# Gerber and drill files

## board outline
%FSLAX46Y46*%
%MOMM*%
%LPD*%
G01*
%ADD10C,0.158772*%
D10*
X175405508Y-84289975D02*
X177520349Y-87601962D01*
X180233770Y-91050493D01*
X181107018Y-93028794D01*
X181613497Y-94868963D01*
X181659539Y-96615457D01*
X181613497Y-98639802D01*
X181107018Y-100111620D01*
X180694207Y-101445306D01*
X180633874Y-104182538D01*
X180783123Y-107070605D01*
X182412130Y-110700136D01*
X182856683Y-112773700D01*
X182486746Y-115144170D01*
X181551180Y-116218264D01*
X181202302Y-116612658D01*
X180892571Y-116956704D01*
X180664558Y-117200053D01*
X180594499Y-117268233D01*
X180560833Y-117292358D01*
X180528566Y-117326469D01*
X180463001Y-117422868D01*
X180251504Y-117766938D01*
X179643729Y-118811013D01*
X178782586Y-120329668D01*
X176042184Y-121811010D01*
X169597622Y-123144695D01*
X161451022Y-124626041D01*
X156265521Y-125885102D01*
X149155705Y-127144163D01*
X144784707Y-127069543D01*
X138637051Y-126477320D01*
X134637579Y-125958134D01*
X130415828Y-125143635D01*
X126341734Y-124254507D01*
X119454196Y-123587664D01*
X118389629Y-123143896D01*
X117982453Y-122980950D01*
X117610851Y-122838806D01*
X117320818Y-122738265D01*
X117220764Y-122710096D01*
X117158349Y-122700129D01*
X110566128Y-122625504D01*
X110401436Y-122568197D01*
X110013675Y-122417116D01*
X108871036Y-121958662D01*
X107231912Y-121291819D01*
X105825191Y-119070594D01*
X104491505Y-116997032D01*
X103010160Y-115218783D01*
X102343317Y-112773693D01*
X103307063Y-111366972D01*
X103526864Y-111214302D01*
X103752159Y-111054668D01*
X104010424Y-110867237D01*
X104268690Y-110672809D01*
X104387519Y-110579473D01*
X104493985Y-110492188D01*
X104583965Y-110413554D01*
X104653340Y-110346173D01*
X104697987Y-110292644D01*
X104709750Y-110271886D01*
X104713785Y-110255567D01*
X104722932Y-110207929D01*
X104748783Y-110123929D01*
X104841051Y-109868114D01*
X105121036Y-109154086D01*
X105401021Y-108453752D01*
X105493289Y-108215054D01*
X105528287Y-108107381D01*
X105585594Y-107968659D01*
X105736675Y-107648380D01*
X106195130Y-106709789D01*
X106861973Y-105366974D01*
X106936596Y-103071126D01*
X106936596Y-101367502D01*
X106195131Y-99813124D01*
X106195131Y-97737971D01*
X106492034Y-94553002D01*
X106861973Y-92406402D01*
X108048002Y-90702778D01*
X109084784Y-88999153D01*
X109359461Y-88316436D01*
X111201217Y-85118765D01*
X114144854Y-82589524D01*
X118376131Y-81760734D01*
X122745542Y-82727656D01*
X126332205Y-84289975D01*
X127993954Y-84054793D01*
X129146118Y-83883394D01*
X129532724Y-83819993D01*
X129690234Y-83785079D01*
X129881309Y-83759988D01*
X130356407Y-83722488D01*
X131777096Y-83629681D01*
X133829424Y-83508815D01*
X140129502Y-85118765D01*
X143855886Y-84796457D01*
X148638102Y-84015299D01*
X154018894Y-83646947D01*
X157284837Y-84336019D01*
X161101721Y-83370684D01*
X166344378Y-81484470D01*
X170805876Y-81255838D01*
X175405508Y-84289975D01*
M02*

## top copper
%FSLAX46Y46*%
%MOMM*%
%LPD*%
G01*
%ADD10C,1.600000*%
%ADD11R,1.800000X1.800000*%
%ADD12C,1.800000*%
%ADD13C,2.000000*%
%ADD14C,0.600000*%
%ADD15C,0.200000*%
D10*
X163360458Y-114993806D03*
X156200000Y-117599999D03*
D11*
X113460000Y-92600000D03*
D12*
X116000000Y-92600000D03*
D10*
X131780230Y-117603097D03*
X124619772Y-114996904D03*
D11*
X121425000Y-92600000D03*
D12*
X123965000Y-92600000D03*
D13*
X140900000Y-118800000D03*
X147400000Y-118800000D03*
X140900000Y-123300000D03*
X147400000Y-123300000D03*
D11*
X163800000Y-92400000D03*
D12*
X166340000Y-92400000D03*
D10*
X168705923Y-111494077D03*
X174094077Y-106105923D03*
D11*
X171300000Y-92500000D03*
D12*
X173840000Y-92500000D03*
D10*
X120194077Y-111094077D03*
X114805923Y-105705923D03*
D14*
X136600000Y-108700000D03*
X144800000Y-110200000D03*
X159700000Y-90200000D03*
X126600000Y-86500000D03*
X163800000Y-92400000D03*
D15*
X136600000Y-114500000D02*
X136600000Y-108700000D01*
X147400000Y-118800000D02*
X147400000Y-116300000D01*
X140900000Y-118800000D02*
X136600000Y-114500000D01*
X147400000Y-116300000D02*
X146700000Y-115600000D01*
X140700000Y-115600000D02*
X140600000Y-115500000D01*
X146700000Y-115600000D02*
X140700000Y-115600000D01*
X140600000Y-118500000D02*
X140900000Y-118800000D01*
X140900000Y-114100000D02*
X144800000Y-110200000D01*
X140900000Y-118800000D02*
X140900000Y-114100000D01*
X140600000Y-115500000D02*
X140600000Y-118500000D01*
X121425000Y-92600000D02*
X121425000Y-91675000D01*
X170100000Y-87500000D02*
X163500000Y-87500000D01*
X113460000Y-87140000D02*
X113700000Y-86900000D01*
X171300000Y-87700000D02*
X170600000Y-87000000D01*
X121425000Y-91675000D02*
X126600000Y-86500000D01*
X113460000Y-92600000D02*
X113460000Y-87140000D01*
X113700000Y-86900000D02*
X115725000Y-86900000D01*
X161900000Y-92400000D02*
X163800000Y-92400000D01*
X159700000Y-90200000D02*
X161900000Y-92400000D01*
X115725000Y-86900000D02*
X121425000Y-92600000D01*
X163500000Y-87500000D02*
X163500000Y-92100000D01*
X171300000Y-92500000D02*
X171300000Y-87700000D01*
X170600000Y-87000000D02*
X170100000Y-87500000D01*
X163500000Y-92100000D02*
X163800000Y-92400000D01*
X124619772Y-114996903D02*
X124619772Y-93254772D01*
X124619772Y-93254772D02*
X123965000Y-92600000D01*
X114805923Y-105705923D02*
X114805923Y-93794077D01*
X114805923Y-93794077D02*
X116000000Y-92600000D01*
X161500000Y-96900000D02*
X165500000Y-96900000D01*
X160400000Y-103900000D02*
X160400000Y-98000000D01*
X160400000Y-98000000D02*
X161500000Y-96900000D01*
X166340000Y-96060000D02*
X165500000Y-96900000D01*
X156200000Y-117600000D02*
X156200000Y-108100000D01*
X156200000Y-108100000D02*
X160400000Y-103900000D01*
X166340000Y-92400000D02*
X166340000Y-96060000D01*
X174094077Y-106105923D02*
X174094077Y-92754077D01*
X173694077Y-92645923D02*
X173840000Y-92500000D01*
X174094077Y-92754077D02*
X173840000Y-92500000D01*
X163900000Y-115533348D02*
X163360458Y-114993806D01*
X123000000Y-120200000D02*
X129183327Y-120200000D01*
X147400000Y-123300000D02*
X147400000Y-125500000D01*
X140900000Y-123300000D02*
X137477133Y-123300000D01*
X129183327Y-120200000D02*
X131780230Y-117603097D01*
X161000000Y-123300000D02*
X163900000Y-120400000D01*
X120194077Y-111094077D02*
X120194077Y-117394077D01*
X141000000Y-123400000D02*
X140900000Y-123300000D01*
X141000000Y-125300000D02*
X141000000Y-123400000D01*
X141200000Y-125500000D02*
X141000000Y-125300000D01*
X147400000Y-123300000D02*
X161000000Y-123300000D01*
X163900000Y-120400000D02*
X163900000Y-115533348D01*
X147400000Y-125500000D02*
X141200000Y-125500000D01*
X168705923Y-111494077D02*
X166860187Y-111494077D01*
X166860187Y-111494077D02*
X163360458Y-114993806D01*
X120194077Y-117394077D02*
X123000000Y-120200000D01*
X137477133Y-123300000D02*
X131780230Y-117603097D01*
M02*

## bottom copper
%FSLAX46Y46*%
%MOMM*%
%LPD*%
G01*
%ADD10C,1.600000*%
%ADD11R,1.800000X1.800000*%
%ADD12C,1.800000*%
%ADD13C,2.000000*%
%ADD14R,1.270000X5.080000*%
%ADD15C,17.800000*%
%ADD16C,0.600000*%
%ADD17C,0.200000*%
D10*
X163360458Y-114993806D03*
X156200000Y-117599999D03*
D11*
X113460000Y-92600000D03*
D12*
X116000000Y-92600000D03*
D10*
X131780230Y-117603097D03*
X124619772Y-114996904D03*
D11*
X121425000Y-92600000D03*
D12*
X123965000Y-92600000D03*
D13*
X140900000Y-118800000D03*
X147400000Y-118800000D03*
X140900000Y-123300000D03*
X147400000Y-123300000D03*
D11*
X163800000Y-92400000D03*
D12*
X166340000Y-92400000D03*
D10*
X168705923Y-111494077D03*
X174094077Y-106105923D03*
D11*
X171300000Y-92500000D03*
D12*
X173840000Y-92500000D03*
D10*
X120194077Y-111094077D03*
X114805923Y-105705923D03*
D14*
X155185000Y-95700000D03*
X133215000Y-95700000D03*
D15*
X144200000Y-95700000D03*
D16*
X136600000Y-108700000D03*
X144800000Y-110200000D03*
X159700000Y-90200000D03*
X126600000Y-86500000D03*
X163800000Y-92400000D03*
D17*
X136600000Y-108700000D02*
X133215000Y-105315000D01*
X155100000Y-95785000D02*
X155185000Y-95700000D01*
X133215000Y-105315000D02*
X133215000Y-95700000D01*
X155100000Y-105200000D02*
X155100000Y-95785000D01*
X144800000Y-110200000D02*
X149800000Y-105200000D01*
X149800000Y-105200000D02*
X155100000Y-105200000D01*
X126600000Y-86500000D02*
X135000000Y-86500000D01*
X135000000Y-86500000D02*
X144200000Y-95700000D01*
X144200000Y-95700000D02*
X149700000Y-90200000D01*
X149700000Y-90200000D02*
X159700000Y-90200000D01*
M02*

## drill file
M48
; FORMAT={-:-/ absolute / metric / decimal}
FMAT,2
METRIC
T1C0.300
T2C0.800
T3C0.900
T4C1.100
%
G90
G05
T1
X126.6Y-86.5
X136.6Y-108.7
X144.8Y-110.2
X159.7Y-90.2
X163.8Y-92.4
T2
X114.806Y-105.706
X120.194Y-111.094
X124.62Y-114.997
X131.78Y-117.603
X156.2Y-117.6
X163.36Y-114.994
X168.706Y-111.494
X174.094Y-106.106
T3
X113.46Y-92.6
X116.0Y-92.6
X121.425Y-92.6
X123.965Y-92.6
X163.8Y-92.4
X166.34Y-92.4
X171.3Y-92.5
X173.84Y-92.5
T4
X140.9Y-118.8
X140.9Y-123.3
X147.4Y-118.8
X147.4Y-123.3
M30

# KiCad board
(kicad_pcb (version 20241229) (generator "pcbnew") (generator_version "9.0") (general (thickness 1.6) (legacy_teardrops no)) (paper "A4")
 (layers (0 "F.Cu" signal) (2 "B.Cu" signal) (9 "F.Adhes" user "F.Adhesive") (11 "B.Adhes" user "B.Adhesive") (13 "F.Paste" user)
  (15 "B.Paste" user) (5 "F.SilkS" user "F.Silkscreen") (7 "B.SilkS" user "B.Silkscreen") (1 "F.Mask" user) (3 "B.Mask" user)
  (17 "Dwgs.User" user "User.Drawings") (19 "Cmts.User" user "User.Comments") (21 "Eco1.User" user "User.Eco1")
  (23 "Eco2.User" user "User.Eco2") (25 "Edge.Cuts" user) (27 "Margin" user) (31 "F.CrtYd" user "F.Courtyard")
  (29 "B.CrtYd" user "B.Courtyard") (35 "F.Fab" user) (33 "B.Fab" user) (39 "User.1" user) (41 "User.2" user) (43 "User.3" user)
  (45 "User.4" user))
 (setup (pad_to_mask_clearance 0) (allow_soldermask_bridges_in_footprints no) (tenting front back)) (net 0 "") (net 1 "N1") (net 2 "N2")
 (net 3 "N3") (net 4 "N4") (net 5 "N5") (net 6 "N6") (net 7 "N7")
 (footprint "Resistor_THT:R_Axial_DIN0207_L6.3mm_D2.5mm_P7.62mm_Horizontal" (layer "F.Cu") (at 163.360458 114.993806 -160)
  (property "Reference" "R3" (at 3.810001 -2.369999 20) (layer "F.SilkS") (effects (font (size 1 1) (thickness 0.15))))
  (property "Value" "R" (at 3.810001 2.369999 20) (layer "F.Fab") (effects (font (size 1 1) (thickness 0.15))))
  (pad "1" thru_hole circle (at 0 0 200) (size 1.6 1.6) (drill 0.8) (layers "*.Cu" "*.Mask") (remove_unused_layers no) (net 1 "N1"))
  (pad "2" thru_hole circle (at 7.62 0 200) (size 1.6 1.6) (drill 0.8) (layers "*.Cu" "*.Mask") (remove_unused_layers no) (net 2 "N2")))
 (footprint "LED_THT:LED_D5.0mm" (layer "F.Cu") (at 113.46 92.6)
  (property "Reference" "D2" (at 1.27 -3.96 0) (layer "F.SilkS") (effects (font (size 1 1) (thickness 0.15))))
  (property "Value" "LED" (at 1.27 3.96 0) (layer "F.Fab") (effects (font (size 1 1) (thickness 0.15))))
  (pad "1" thru_hole rect (at 0 0) (size 1.8 1.8) (drill 0.9) (layers "*.Cu" "*.Mask") (remove_unused_layers no) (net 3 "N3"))
  (pad "2" thru_hole circle (at 2.54 0) (size 1.8 1.8) (drill 0.9) (layers "*.Cu" "*.Mask") (remove_unused_layers no) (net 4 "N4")))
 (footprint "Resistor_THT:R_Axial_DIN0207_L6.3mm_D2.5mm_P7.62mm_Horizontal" (layer "F.Cu") (at 131.78023 117.603097 160)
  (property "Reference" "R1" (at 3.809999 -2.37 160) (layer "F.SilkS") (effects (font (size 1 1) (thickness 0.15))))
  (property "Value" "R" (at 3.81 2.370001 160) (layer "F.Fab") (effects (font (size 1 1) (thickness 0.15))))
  (pad "1" thru_hole circle (at 0 0 160) (size 1.6 1.6) (drill 0.8) (layers "*.Cu" "*.Mask") (remove_unused_layers no) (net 1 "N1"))
  (pad "2" thru_hole circle (at 7.62 0 160) (size 1.6 1.6) (drill 0.8) (layers "*.Cu" "*.Mask") (remove_unused_layers no) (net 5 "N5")))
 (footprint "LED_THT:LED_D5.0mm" (layer "F.Cu") (at 121.425 92.6)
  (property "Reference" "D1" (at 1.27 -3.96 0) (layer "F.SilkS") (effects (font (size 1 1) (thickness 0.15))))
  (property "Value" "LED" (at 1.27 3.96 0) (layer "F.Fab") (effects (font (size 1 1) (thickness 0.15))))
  (pad "1" thru_hole rect (at 0 0) (size 1.8 1.8) (drill 0.9) (layers "*.Cu" "*.Mask") (remove_unused_layers no) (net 3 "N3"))
  (pad "2" thru_hole circle (at 2.54 0) (size 1.8 1.8) (drill 0.9) (layers "*.Cu" "*.Mask") (remove_unused_layers no) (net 5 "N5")))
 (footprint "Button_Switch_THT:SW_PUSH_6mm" (layer "F.Cu") (at 140.9 118.8)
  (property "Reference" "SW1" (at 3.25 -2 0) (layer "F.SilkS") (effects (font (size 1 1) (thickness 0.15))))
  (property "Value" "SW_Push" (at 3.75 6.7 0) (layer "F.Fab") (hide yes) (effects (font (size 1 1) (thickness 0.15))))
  (pad "1" thru_hole circle (at 0 0 90) (size 2 2) (drill 1.1) (layers "*.Cu" "*.Mask") (remove_unused_layers no) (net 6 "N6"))
  (pad "1" thru_hole circle (at 6.5 0 90) (size 2 2) (drill 1.1) (layers "*.Cu" "*.Mask") (remove_unused_layers no) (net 6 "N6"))
  (pad "2" thru_hole circle (at 0 4.5 90) (size 2 2) (drill 1.1) (layers "*.Cu" "*.Mask") (remove_unused_layers no) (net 1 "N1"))
  (pad "2" thru_hole circle (at 6.5 4.5 90) (size 2 2) (drill 1.1) (layers "*.Cu" "*.Mask") (remove_unused_layers no) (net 1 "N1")))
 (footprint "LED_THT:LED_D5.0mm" (layer "F.Cu") (at 163.8 92.4)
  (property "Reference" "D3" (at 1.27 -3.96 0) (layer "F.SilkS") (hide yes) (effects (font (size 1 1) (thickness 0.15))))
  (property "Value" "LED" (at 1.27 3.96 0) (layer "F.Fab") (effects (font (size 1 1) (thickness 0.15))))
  (pad "1" thru_hole rect (at 0 0) (size 1.8 1.8) (drill 0.9) (layers "*.Cu" "*.Mask") (remove_unused_layers no) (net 3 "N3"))
  (pad "2" thru_hole circle (at 2.54 0) (size 1.8 1.8) (drill 0.9) (layers "*.Cu" "*.Mask") (remove_unused_layers no) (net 2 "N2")))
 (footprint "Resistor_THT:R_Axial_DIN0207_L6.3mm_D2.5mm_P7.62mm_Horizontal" (layer "F.Cu") (at 168.705923 111.494077 45)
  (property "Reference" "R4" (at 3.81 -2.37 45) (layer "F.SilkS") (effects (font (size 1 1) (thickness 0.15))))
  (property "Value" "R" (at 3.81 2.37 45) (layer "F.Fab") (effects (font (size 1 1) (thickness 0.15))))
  (pad "1" thru_hole circle (at 0 0 45) (size 1.6 1.6) (drill 0.8) (layers "*.Cu" "*.Mask") (remove_unused_layers no) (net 1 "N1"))
  (pad "2" thru_hole circle (at 7.62 0 45) (size 1.6 1.6) (drill 0.8) (layers "*.Cu" "*.Mask") (remove_unused_layers no) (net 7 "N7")))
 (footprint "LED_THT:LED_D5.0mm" (layer "F.Cu") (at 171.3 92.5)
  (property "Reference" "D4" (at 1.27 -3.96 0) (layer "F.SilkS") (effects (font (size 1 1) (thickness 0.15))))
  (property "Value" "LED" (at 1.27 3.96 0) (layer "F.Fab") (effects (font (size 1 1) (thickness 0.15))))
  (pad "1" thru_hole rect (at 0 0) (size 1.8 1.8) (drill 0.9) (layers "*.Cu" "*.Mask") (remove_unused_layers no) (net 3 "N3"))
  (pad "2" thru_hole circle (at 2.54 0) (size 1.8 1.8) (drill 0.9) (layers "*.Cu" "*.Mask") (remove_unused_layers no) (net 7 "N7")))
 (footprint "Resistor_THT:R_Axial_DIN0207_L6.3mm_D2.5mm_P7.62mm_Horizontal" (layer "F.Cu") (at 120.194077 111.094077 135)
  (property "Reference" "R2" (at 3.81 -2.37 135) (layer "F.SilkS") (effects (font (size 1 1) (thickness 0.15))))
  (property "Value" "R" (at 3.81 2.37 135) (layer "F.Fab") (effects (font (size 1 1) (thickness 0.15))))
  (pad "1" thru_hole circle (at 0 0 135) (size 1.6 1.6) (drill 0.8) (layers "*.Cu" "*.Mask") (remove_unused_layers no) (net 1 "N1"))
  (pad "2" thru_hole circle (at 7.62 0 135) (size 1.6 1.6) (drill 0.8) (layers "*.Cu" "*.Mask") (remove_unused_layers no) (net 4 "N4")))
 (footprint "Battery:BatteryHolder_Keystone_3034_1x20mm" (layer "B.Cu") (at 144.2 95.7 180)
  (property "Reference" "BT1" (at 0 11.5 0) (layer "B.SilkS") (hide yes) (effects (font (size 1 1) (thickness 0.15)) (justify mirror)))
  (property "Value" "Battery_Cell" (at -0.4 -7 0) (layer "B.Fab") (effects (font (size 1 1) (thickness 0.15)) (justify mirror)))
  (pad "1" smd rect (at -10.985 0 180) (size 1.27 5.08) (layers "B.Cu" "B.Mask" "B.Paste") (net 6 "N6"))
  (pad "1" smd rect (at 10.985 0 180) (size 1.27 5.08) (layers "B.Cu" "B.Mask" "B.Paste") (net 6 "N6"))
  (pad "2" smd circle (at 0 0 180) (size 17.8 17.8) (layers "B.Cu" "B.Mask") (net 3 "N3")))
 (gr_poly
  (pts (xy 175.405508 84.289975) (xy 177.520349 87.601962) (xy 180.23377 91.050493) (xy 181.107018 93.028794) (xy 181.613497 94.868963)
   (xy 181.659539 96.615457) (xy 181.613497 98.639802) (xy 181.107018 100.11162) (xy 180.694207 101.445306) (xy 180.633874 104.182538)
   (xy 180.783123 107.070605) (xy 182.41213 110.700136) (xy 182.856683 112.7737) (xy 182.486746 115.14417) (xy 181.55118 116.218264)
   (xy 181.202302 116.612658) (xy 180.892571 116.956704) (xy 180.664558 117.200053) (xy 180.594499 117.268233) (xy 180.560833 117.292358)
   (xy 180.528566 117.326469) (xy 180.463001 117.422868) (xy 180.251504 117.766938) (xy 179.643729 118.811013) (xy 178.782586 120.329668)
   (xy 176.042184 121.81101) (xy 169.597622 123.144695) (xy 161.451022 124.626041) (xy 156.265521 125.885102) (xy 149.155705 127.144163)
   (xy 144.784707 127.069543) (xy 138.637051 126.47732) (xy 134.637579 125.958134) (xy 130.415828 125.143635) (xy 126.341734 124.254507)
   (xy 119.454196 123.587664) (xy 118.389629 123.143896) (xy 117.982453 122.98095) (xy 117.610851 122.838806) (xy 117.320818 122.738265)
   (xy 117.220764 122.710096) (xy 117.158349 122.700129) (xy 110.566128 122.625504) (xy 110.401436 122.568197) (xy 110.013675 122.417116)
   (xy 108.871036 121.958662) (xy 107.231912 121.291819) (xy 105.825191 119.070594) (xy 104.491505 116.997032) (xy 103.01016 115.218783)
   (xy 102.343317 112.773693) (xy 103.307063 111.366972) (xy 103.526864 111.214302) (xy 103.752159 111.054668) (xy 104.010424 110.867237)
   (xy 104.26869 110.672809) (xy 104.387519 110.579473) (xy 104.493985 110.492188) (xy 104.583965 110.413554) (xy 104.65334 110.346173)
   (xy 104.697987 110.292644) (xy 104.70975 110.271886) (xy 104.713785 110.255567) (xy 104.722932 110.207929) (xy 104.748783 110.123929)
   (xy 104.841051 109.868114) (xy 105.121036 109.154086) (xy 105.401021 108.453752) (xy 105.493289 108.215054) (xy 105.528287 108.107381)
   (xy 105.585594 107.968659) (xy 105.736675 107.64838) (xy 106.19513 106.709789) (xy 106.861973 105.366974) (xy 106.936596 103.071126)
   (xy 106.936596 101.367502) (xy 106.195131 99.813124) (xy 106.195131 97.737971) (xy 106.492034 94.553002) (xy 106.861973 92.406402)
   (xy 108.048002 90.702778) (xy 109.084784 88.999153) (xy 109.359461 88.316436) (xy 111.201217 85.118765) (xy 114.144854 82.589524)
   (xy 118.376131 81.760734) (xy 122.745542 82.727656) (xy 126.332205 84.289975) (xy 127.993954 84.054793) (xy 129.146118 83.883394)
   (xy 129.532724 83.819993) (xy 129.690234 83.785079) (xy 129.881309 83.759988) (xy 130.356407 83.722488) (xy 131.777096 83.629681)
   (xy 133.829424 83.508815) (xy 140.129502 85.118765) (xy 143.855886 84.796457) (xy 148.638102 84.015299) (xy 154.018894 83.646947)
   (xy 157.284837 84.336019) (xy 161.101721 83.370684) (xy 166.344378 81.48447) (xy 170.805876 81.255838))
  (stroke (width 0.158772) (type solid)) (fill no) (layer "Edge.Cuts"))
 (segment (start 136.6 114.5) (end 136.6 108.7) (width 0.2) (layer "F.Cu") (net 6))
 (segment (start 147.4 118.8) (end 147.4 116.3) (width 0.2) (layer "F.Cu") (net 6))
 (segment (start 140.9 118.8) (end 136.6 114.5) (width 0.2) (layer "F.Cu") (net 6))
 (segment (start 147.4 116.3) (end 146.7 115.6) (width 0.2) (layer "F.Cu") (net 6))
 (segment (start 140.7 115.6) (end 140.6 115.5) (width 0.2) (layer "F.Cu") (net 6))
 (segment (start 146.7 115.6) (end 140.7 115.6) (width 0.2) (layer "F.Cu") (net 6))
 (segment (start 140.6 118.5) (end 140.9 118.8) (width 0.2) (layer "F.Cu") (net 6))
 (segment (start 140.9 114.1) (end 144.8 110.2) (width 0.2) (layer "F.Cu") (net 6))
 (segment (start 140.9 118.8) (end 140.9 114.1) (width 0.2) (layer "F.Cu") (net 6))
 (segment (start 140.6 115.5) (end 140.6 118.5) (width 0.2) (layer "F.Cu") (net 6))
 (via (at 136.6 108.7) (size 0.6) (drill 0.3) (layers "F.Cu" "B.Cu") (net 6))
 (via (at 144.8 110.2) (size 0.6) (drill 0.3) (layers "F.Cu" "B.Cu") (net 6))
 (segment (start 136.6 108.7) (end 133.215 105.315) (width 0.2) (layer "B.Cu") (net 6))
 (segment (start 155.1 95.785) (end 155.185 95.7) (width 0.2) (layer "B.Cu") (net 6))
 (segment (start 133.215 105.315) (end 133.215 95.7) (width 0.2) (layer "B.Cu") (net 6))
 (segment (start 155.1 105.2) (end 155.1 95.785) (width 0.2) (layer "B.Cu") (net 6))
 (segment (start 144.8 110.2) (end 149.8 105.2) (width 0.2) (layer "B.Cu") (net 6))
 (segment (start 149.8 105.2) (end 155.1 105.2) (width 0.2) (layer "B.Cu") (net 6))
 (segment (start 121.425 92.6) (end 121.425 91.675) (width 0.2) (layer "F.Cu") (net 3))
 (segment (start 170.1 87.5) (end 163.5 87.5) (width 0.2) (layer "F.Cu") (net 3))
 (segment (start 113.46 87.14) (end 113.7 86.9) (width 0.2) (layer "F.Cu") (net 3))
 (segment (start 171.3 87.7) (end 170.6 87) (width 0.2) (layer "F.Cu") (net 3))
 (segment (start 121.425 91.675) (end 126.6 86.5) (width 0.2) (layer "F.Cu") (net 3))
 (segment (start 113.46 92.6) (end 113.46 87.14) (width 0.2) (layer "F.Cu") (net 3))
 (segment (start 113.7 86.9) (end 115.725 86.9) (width 0.2) (layer "F.Cu") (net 3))
 (segment (start 161.9 92.4) (end 163.8 92.4) (width 0.2) (layer "F.Cu") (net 3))
 (segment (start 159.7 90.2) (end 161.9 92.4) (width 0.2) (layer "F.Cu") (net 3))
 (segment (start 115.725 86.9) (end 121.425 92.6) (width 0.2) (layer "F.Cu") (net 3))
 (segment (start 163.5 87.5) (end 163.5 92.1) (width 0.2) (layer "F.Cu") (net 3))
 (segment (start 171.3 92.5) (end 171.3 87.7) (width 0.2) (layer "F.Cu") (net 3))
 (segment (start 170.6 87) (end 170.1 87.5) (width 0.2) (layer "F.Cu") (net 3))
 (segment (start 163.5 92.1) (end 163.8 92.4) (width 0.2) (layer "F.Cu") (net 3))
 (via (at 159.7 90.2) (size 0.6) (drill 0.3) (layers "F.Cu" "B.Cu") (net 3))
 (via (at 126.6 86.5) (size 0.6) (drill 0.3) (layers "F.Cu" "B.Cu") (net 3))
 (via (at 163.8 92.4) (size 0.6) (drill 0.3) (layers "F.Cu" "B.Cu") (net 3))
 (segment (start 126.6 86.5) (end 135 86.5) (width 0.2) (layer "B.Cu") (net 3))
 (segment (start 135 86.5) (end 144.2 95.7) (width 0.2) (layer "B.Cu") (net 3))
 (segment (start 144.2 95.7) (end 149.7 90.2) (width 0.2) (layer "B.Cu") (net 3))
 (segment (start 149.7 90.2) (end 159.7 90.2) (width 0.2) (layer "B.Cu") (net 3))
 (segment (start 124.619772 114.996903) (end 124.619772 93.254772) (width 0.2) (layer "F.Cu") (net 5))
 (segment (start 124.619772 93.254772) (end 123.965 92.6) (width 0.2) (layer "F.Cu") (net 5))
 (segment (start 114.805923 105.705923) (end 114.805923 93.794077) (width 0.2) (layer "F.Cu") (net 4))
 (segment (start 114.805923 93.794077) (end 116 92.6) (width 0.2) (layer "F.Cu") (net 4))
 (segment (start 161.5 96.9) (end 165.5 96.9) (width 0.2) (layer "F.Cu") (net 2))
 (segment (start 160.4 103.9) (end 160.4 98) (width 0.2) (layer "F.Cu") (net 2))
 (segment (start 160.4 98) (end 161.5 96.9) (width 0.2) (layer "F.Cu") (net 2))
 (segment (start 166.34 96.06) (end 165.5 96.9) (width 0.2) (layer "F.Cu") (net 2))
 (segment (start 156.2 117.6) (end 156.2 108.1) (width 0.2) (layer "F.Cu") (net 2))
 (segment (start 156.2 108.1) (end 160.4 103.9) (width 0.2) (layer "F.Cu") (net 2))
 (segment (start 166.34 92.4) (end 166.34 96.06) (width 0.2) (layer "F.Cu") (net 2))
 (segment (start 174.094077 106.105923) (end 174.094077 92.754077) (width 0.2) (layer "F.Cu") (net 7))
 (segment (start 173.694077 92.645923) (end 173.84 92.5) (width 0.2) (layer "F.Cu") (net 7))
 (segment (start 174.094077 92.754077) (end 173.84 92.5) (width 0.2) (layer "F.Cu") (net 7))
 (segment (start 163.9 115.533348) (end 163.360458 114.993806) (width 0.2) (layer "F.Cu") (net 1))
 (segment (start 123 120.2) (end 129.183327 120.2) (width 0.2) (layer "F.Cu") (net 1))
 (segment (start 147.4 123.3) (end 147.4 125.5) (width 0.2) (layer "F.Cu") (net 1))
 (segment (start 140.9 123.3) (end 137.477133 123.3) (width 0.2) (layer "F.Cu") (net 1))
 (segment (start 129.183327 120.2) (end 131.78023 117.603097) (width 0.2) (layer "F.Cu") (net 1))
 (segment (start 161 123.3) (end 163.9 120.4) (width 0.2) (layer "F.Cu") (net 1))
 (segment (start 120.194077 111.094077) (end 120.194077 117.394077) (width 0.2) (layer "F.Cu") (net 1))
 (segment (start 141 123.4) (end 140.9 123.3) (width 0.2) (layer "F.Cu") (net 1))
 (segment (start 141 125.3) (end 141 123.4) (width 0.2) (layer "F.Cu") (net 1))
 (segment (start 141.2 125.5) (end 141 125.3) (width 0.2) (layer "F.Cu") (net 1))
 (segment (start 147.4 123.3) (end 161 123.3) (width 0.2) (layer "F.Cu") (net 1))
 (segment (start 163.9 120.4) (end 163.9 115.533348) (width 0.2) (layer "F.Cu") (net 1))
 (segment (start 147.4 125.5) (end 141.2 125.5) (width 0.2) (layer "F.Cu") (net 1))
 (segment (start 168.705923 111.494077) (end 166.860187 111.494077) (width 0.2) (layer "F.Cu") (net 1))
 (segment (start 166.860187 111.494077) (end 163.360458 114.993806) (width 0.2) (layer "F.Cu") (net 1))
 (segment (start 120.194077 117.394077) (end 123 120.2) (width 0.2) (layer "F.Cu") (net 1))
 (segment (start 137.477133 123.3) (end 131.78023 117.603097) (width 0.2) (layer "F.Cu") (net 1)))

